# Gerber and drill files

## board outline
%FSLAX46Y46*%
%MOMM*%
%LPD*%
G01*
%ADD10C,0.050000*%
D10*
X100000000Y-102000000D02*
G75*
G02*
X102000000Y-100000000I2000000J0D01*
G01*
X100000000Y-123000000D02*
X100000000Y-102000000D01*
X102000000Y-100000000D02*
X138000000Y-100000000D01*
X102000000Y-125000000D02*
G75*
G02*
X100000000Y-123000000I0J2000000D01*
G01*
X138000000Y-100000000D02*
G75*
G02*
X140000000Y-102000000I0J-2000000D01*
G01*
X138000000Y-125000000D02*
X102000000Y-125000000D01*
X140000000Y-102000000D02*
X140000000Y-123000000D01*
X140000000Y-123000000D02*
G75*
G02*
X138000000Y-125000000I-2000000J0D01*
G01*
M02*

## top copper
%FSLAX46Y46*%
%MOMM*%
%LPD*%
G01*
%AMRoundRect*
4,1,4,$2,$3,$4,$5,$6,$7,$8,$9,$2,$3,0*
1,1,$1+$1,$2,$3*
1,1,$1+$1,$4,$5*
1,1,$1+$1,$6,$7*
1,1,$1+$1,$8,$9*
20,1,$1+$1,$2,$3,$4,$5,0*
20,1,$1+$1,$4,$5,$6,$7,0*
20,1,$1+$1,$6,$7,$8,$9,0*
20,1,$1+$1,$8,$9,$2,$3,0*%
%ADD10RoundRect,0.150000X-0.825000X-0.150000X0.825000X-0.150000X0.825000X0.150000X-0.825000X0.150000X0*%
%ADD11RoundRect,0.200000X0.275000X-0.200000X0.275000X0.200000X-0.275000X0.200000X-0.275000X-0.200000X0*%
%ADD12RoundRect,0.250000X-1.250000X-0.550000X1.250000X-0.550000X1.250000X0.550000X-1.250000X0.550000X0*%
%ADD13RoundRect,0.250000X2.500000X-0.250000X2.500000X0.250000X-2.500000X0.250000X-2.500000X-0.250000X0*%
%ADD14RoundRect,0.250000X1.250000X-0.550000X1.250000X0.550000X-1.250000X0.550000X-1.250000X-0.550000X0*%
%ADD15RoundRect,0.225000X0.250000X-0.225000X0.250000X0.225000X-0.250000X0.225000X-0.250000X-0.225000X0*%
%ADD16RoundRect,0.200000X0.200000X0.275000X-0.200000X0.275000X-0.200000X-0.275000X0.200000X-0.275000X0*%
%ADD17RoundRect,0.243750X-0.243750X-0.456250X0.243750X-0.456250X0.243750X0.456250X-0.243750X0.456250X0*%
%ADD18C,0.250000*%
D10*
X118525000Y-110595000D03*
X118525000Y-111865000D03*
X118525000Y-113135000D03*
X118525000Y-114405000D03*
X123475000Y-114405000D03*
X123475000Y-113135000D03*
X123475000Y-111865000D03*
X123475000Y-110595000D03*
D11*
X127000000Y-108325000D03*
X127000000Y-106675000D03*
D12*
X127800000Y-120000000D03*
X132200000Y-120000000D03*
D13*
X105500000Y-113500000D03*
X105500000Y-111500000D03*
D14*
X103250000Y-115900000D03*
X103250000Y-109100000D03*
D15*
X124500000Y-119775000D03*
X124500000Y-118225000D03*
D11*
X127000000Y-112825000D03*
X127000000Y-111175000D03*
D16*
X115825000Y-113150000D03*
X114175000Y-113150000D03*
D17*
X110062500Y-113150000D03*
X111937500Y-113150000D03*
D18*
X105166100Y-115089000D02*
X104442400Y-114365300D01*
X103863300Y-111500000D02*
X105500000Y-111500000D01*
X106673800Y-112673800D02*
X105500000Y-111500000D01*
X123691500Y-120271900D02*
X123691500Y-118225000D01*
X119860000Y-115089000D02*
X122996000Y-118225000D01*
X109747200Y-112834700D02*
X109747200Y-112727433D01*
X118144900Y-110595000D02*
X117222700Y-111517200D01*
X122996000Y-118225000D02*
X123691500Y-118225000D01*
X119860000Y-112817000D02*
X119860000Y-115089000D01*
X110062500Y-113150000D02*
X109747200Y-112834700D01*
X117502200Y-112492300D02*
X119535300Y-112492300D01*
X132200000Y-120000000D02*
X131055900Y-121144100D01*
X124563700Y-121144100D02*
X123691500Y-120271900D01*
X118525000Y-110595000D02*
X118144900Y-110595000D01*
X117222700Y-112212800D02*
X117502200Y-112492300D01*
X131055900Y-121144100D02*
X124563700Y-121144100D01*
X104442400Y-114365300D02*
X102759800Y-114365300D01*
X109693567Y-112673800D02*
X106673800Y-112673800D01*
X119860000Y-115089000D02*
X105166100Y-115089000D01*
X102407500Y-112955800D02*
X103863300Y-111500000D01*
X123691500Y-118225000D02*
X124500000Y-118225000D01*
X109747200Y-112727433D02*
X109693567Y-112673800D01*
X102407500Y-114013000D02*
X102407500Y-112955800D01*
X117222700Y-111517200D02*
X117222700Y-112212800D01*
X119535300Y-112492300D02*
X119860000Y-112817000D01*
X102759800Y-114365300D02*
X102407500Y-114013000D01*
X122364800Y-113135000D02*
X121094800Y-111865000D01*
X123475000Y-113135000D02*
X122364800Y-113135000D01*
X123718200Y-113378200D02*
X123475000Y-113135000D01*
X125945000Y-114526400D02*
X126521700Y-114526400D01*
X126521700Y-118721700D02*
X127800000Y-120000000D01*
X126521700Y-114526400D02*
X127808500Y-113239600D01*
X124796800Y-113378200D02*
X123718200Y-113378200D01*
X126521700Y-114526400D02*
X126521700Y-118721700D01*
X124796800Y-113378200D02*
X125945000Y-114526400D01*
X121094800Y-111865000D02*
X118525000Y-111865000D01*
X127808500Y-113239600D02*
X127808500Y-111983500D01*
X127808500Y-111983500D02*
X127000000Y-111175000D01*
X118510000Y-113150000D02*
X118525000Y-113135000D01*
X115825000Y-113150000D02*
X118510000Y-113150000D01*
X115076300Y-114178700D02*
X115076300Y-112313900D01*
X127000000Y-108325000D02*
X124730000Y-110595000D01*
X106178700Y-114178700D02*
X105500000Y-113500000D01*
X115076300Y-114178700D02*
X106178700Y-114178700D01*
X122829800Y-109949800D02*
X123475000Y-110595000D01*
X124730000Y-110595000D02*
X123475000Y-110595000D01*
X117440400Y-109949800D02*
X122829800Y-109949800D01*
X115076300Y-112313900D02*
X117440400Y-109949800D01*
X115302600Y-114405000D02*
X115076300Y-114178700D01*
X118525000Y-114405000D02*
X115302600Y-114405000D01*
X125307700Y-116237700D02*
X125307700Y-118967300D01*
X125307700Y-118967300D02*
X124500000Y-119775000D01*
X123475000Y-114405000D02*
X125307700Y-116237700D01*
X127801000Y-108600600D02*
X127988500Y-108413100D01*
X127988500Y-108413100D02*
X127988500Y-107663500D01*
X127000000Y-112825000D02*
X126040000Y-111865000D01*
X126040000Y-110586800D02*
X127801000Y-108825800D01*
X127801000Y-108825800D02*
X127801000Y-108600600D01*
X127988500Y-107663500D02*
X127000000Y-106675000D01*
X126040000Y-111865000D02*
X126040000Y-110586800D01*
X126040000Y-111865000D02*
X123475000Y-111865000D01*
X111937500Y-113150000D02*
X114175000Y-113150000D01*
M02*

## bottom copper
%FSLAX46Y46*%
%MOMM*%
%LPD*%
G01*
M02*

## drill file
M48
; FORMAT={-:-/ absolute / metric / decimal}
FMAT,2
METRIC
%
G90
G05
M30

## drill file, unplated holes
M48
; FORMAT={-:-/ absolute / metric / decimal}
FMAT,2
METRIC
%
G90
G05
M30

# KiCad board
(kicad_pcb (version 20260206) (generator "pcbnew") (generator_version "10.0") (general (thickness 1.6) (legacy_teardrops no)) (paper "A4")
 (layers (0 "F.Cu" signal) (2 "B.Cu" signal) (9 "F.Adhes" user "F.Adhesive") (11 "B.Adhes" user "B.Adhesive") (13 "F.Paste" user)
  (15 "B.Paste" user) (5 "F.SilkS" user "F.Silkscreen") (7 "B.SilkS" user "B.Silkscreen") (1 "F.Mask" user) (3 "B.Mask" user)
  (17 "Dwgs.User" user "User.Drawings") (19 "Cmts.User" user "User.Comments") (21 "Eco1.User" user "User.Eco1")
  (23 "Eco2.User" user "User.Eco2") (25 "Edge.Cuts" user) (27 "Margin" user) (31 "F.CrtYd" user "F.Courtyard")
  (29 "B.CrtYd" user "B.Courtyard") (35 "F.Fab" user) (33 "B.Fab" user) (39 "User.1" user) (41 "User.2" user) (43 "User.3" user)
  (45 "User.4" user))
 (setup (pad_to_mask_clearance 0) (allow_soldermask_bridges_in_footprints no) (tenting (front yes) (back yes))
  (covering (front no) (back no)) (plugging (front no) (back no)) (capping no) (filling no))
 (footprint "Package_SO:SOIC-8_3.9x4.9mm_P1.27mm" (layer "F.Cu") (at 121 112.5)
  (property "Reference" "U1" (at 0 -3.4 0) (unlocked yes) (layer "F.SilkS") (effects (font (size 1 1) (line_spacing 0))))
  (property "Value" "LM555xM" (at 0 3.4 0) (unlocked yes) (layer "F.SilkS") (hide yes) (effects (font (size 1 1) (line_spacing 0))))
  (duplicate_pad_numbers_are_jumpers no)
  (pad "1" smd roundrect (at -2.475 -1.905) (size 1.95 0.6) (layers "F.Cu" "F.Mask" "F.Paste") (roundrect_rratio 0.25) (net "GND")
   (zone_connect 0))
  (pad "2" smd roundrect (at -2.475 -0.635) (size 1.95 0.6) (layers "F.Cu" "F.Mask" "F.Paste") (roundrect_rratio 0.25)
   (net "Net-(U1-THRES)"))
  (pad "3" smd roundrect (at -2.475 0.635) (size 1.95 0.6) (layers "F.Cu" "F.Mask" "F.Paste") (roundrect_rratio 0.25) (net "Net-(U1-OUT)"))
  (pad "4" smd roundrect (at -2.475 1.905) (size 1.95 0.6) (layers "F.Cu" "F.Mask" "F.Paste") (roundrect_rratio 0.25) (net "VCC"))
  (pad "5" smd roundrect (at 2.475 1.905) (size 1.95 0.6) (layers "F.Cu" "F.Mask" "F.Paste") (roundrect_rratio 0.25) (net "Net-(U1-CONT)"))
  (pad "6" smd roundrect (at 2.475 0.635) (size 1.95 0.6) (layers "F.Cu" "F.Mask" "F.Paste") (roundrect_rratio 0.25) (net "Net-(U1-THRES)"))
  (pad "7" smd roundrect (at 2.475 -0.635) (size 1.95 0.6) (layers "F.Cu" "F.Mask" "F.Paste") (roundrect_rratio 0.25) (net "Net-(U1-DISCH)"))
  (pad "8" smd roundrect (at 2.475 -1.905) (size 1.95 0.6) (layers "F.Cu" "F.Mask" "F.Paste") (roundrect_rratio 0.25) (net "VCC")))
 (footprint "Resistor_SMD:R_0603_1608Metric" (layer "F.Cu") (at 127 107.5 90)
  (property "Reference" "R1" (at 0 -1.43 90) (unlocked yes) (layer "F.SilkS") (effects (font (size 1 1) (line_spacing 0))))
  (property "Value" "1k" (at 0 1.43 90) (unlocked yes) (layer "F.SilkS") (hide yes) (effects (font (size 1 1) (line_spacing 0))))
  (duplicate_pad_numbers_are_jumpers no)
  (pad "1" smd roundrect (at -0.825 0 90) (size 0.8 0.95) (layers "F.Cu" "F.Mask" "F.Paste") (roundrect_rratio 0.25) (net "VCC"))
  (pad "2" smd roundrect (at 0.825 0 90) (size 0.8 0.95) (layers "F.Cu" "F.Mask" "F.Paste") (roundrect_rratio 0.25) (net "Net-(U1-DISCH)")))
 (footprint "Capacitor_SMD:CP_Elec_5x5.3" (layer "F.Cu") (at 130 120)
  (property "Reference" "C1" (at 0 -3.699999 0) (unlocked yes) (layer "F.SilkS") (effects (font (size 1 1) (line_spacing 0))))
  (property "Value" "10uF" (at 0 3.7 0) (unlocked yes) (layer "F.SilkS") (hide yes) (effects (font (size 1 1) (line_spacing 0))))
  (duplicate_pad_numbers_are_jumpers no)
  (pad "1" smd roundrect (at -2.2 0) (size 3 1.6) (layers "F.Cu" "F.Mask" "F.Paste") (roundrect_rratio 0.15625) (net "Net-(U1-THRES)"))
  (pad "2" smd roundrect (at 2.2 0) (size 3 1.6) (layers "F.Cu" "F.Mask" "F.Paste") (roundrect_rratio 0.15625) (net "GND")))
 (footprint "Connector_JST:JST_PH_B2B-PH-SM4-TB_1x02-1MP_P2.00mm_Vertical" (layer "F.Cu") (at 105 112.5 90)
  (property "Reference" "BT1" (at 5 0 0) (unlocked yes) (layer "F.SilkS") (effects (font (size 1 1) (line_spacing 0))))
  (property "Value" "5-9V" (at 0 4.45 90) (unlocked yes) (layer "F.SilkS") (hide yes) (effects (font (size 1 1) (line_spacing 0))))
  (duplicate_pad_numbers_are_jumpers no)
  (pad "1" smd roundrect (at -1 0.5 90) (size 1 5.5) (layers "F.Cu" "F.Mask" "F.Paste") (roundrect_rratio 0.25) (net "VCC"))
  (pad "2" smd roundrect (at 1 0.5 90) (size 1 5.5) (layers "F.Cu" "F.Mask" "F.Paste") (roundrect_rratio 0.25) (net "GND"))
  (pad "MP" smd roundrect (at -3.4 -1.75 90) (size 1.6 3) (layers "F.Cu" "F.Mask" "F.Paste") (roundrect_rratio 0.15625))
  (pad "MP" smd roundrect (at 3.4 -1.75 90) (size 1.6 3) (layers "F.Cu" "F.Mask" "F.Paste") (roundrect_rratio 0.15625)))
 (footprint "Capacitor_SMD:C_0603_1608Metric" (layer "F.Cu") (at 124.5 119 90)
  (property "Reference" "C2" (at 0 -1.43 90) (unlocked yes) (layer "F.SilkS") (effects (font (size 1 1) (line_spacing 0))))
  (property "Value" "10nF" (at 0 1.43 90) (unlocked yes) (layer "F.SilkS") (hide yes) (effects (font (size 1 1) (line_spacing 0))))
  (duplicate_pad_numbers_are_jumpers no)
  (pad "1" smd roundrect (at -0.775 0 90) (size 0.9 0.95) (layers "F.Cu" "F.Mask" "F.Paste") (roundrect_rratio 0.25) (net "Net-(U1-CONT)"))
  (pad "2" smd roundrect (at 0.775 0 90) (size 0.9 0.95) (layers "F.Cu" "F.Mask" "F.Paste") (roundrect_rratio 0.25) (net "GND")))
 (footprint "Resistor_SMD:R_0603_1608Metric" (layer "F.Cu") (at 127 112 90)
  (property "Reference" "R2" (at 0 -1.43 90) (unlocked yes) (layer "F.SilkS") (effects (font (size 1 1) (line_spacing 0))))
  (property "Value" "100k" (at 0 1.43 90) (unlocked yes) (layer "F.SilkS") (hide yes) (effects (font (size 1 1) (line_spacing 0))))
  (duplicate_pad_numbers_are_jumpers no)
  (pad "1" smd roundrect (at -0.825 0 90) (size 0.8 0.95) (layers "F.Cu" "F.Mask" "F.Paste") (roundrect_rratio 0.25) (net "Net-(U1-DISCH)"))
  (pad "2" smd roundrect (at 0.825 0 90) (size 0.8 0.95) (layers "F.Cu" "F.Mask" "F.Paste") (roundrect_rratio 0.25) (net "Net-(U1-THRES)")))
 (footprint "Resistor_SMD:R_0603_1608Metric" (layer "F.Cu") (at 115 113.15 180)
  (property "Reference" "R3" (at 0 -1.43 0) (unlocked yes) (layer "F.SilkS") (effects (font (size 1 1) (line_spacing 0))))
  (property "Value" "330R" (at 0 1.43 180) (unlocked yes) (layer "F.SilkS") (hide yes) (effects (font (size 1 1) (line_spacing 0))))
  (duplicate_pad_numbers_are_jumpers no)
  (pad "1" smd roundrect (at -0.825 0 180) (size 0.8 0.95) (layers "F.Cu" "F.Mask" "F.Paste") (roundrect_rratio 0.25) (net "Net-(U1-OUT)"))
  (pad "2" smd roundrect (at 0.825 0 180) (size 0.8 0.95) (layers "F.Cu" "F.Mask" "F.Paste") (roundrect_rratio 0.25) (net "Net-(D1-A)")))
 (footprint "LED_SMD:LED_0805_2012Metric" (layer "F.Cu") (at 111 113.15)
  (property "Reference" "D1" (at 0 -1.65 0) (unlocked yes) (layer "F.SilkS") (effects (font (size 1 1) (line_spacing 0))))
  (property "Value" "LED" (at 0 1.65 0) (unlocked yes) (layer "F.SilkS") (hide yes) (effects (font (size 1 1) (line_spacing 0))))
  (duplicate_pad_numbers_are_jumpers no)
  (pad "1" smd roundrect (at -0.9375 0) (size 0.975 1.4) (layers "F.Cu" "F.Mask" "F.Paste") (roundrect_rratio 0.25) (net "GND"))
  (pad "2" smd roundrect (at 0.9375 0) (size 0.975 1.4) (layers "F.Cu" "F.Mask" "F.Paste") (roundrect_rratio 0.25) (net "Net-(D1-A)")))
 (gr_arc (start 100 102) (mid 100.585786 100.585786) (end 102 100) (stroke (width 0.05) (type default)) (layer "Edge.Cuts"))
 (gr_line (start 100 123) (end 100 102) (stroke (width 0.05) (type default)) (layer "Edge.Cuts"))
 (gr_line (start 102 100) (end 138 100) (stroke (width 0.05) (type default)) (layer "Edge.Cuts"))
 (gr_arc (start 102 125) (mid 100.585786 124.414213) (end 100 123) (stroke (width 0.05) (type default)) (layer "Edge.Cuts"))
 (gr_arc (start 138 100) (mid 139.414213 100.585786) (end 140 102) (stroke (width 0.05) (type default)) (layer "Edge.Cuts"))
 (gr_line (start 138 125) (end 102 125) (stroke (width 0.05) (type default)) (layer "Edge.Cuts"))
 (gr_line (start 140 102) (end 140 123) (stroke (width 0.05) (type default)) (layer "Edge.Cuts"))
 (gr_arc (start 140 123) (mid 139.414213 124.414213) (end 138 125) (stroke (width 0.05) (type default)) (layer "Edge.Cuts"))
 (segment (start 105.1661 115.089) (end 104.4424 114.3653) (width 0.25) (layer "F.Cu") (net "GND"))
 (segment (start 103.8633 111.5) (end 105.5 111.5) (width 0.25) (layer "F.Cu") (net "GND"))
 (segment (start 106.6738 112.6738) (end 105.5 111.5) (width 0.25) (layer "F.Cu") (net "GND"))
 (segment (start 123.6915 120.2719) (end 123.6915 118.225) (width 0.25) (layer "F.Cu") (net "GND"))
 (segment (start 119.86 115.089) (end 122.996 118.225) (width 0.25) (layer "F.Cu") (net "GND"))
 (segment (start 109.7472 112.8347) (end 109.747200 112.727433) (width 0.25) (layer "F.Cu") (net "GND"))
 (segment (start 118.1449 110.595) (end 117.2227 111.5172) (width 0.25) (layer "F.Cu") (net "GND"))
 (segment (start 122.996 118.225) (end 123.6915 118.225) (width 0.25) (layer "F.Cu") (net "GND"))
 (segment (start 119.86 112.817) (end 119.86 115.089) (width 0.25) (layer "F.Cu") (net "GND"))
 (segment (start 110.0625 113.15) (end 109.7472 112.8347) (width 0.25) (layer "F.Cu") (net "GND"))
 (segment (start 117.5022 112.4923) (end 119.5353 112.4923) (width 0.25) (layer "F.Cu") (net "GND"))
 (segment (start 132.2 120) (end 131.0559 121.1441) (width 0.25) (layer "F.Cu") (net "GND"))
 (segment (start 124.5637 121.1441) (end 123.6915 120.2719) (width 0.25) (layer "F.Cu") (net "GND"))
 (segment (start 118.525 110.595) (end 118.1449 110.595) (width 0.25) (layer "F.Cu") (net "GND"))
 (segment (start 117.2227 112.2128) (end 117.5022 112.4923) (width 0.25) (layer "F.Cu") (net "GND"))
 (segment (start 131.0559 121.1441) (end 124.5637 121.1441) (width 0.25) (layer "F.Cu") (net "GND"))
 (segment (start 104.4424 114.3653) (end 102.7598 114.3653) (width 0.25) (layer "F.Cu") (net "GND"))
 (segment (start 109.693567 112.673800) (end 106.6738 112.6738) (width 0.25) (layer "F.Cu") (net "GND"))
 (segment (start 119.86 115.089) (end 105.1661 115.089) (width 0.25) (layer "F.Cu") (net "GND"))
 (segment (start 102.4075 112.9558) (end 103.8633 111.5) (width 0.25) (layer "F.Cu") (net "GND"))
 (segment (start 123.6915 118.225) (end 124.5 118.225) (width 0.25) (layer "F.Cu") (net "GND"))
 (segment (start 102.4075 114.013) (end 102.4075 112.9558) (width 0.25) (layer "F.Cu") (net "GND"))
 (segment (start 117.2227 111.5172) (end 117.2227 112.2128) (width 0.25) (layer "F.Cu") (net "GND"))
 (segment (start 119.5353 112.4923) (end 119.86 112.817) (width 0.25) (layer "F.Cu") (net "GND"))
 (segment (start 102.7598 114.3653) (end 102.4075 114.013) (width 0.25) (layer "F.Cu") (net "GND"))
 (segment (start 122.3648 113.135) (end 121.0948 111.865) (width 0.25) (layer "F.Cu") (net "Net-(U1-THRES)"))
 (segment (start 123.475 113.135) (end 122.3648 113.135) (width 0.25) (layer "F.Cu") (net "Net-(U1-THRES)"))
 (segment (start 123.7182 113.3782) (end 123.475 113.135) (width 0.25) (layer "F.Cu") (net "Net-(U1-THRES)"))
 (segment (start 125.945 114.5264) (end 126.5217 114.5264) (width 0.25) (layer "F.Cu") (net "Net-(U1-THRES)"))
 (segment (start 126.5217 118.7217) (end 127.8 120) (width 0.25) (layer "F.Cu") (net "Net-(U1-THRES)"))
 (segment (start 126.5217 114.5264) (end 127.8085 113.2396) (width 0.25) (layer "F.Cu") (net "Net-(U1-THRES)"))
 (segment (start 124.7968 113.3782) (end 123.7182 113.3782) (width 0.25) (layer "F.Cu") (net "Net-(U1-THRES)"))
 (segment (start 126.5217 114.5264) (end 126.5217 118.7217) (width 0.25) (layer "F.Cu") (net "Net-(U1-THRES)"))
 (segment (start 124.7968 113.3782) (end 125.945 114.5264) (width 0.25) (layer "F.Cu") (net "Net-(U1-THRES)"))
 (segment (start 121.0948 111.865) (end 118.525 111.865) (width 0.25) (layer "F.Cu") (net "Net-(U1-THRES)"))
 (segment (start 127.8085 113.2396) (end 127.8085 111.9835) (width 0.25) (layer "F.Cu") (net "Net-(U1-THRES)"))
 (segment (start 127.8085 111.9835) (end 127 111.175) (width 0.25) (layer "F.Cu") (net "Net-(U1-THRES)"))
 (segment (start 118.51 113.15) (end 118.525 113.135) (width 0.25) (layer "F.Cu") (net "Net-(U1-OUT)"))
 (segment (start 115.825 113.15) (end 118.51 113.15) (width 0.25) (layer "F.Cu") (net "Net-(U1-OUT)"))
 (segment (start 115.0763 114.1787) (end 115.0763 112.3139) (width 0.25) (layer "F.Cu") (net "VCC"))
 (segment (start 127 108.325) (end 124.73 110.595) (width 0.25) (layer "F.Cu") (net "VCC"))
 (segment (start 106.1787 114.1787) (end 105.5 113.5) (width 0.25) (layer "F.Cu") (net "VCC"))
 (segment (start 115.0763 114.1787) (end 106.1787 114.1787) (width 0.25) (layer "F.Cu") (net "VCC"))
 (segment (start 122.8298 109.9498) (end 123.475 110.595) (width 0.25) (layer "F.Cu") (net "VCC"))
 (segment (start 124.73 110.595) (end 123.475 110.595) (width 0.25) (layer "F.Cu") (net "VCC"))
 (segment (start 117.4404 109.9498) (end 122.8298 109.9498) (width 0.25) (layer "F.Cu") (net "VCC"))
 (segment (start 115.0763 112.3139) (end 117.4404 109.9498) (width 0.25) (layer "F.Cu") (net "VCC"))
 (segment (start 115.3026 114.405) (end 115.0763 114.1787) (width 0.25) (layer "F.Cu") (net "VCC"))
 (segment (start 118.525 114.405) (end 115.3026 114.405) (width 0.25) (layer "F.Cu") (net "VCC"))
 (segment (start 125.3077 116.2377) (end 125.3077 118.9673) (width 0.25) (layer "F.Cu") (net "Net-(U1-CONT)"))
 (segment (start 125.3077 118.9673) (end 124.5 119.775) (width 0.25) (layer "F.Cu") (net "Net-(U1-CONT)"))
 (segment (start 123.475 114.405) (end 125.3077 116.2377) (width 0.25) (layer "F.Cu") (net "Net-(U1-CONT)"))
 (segment (start 127.801 108.6006) (end 127.9885 108.4131) (width 0.25) (layer "F.Cu") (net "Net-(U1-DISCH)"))
 (segment (start 127.9885 108.4131) (end 127.9885 107.6635) (width 0.25) (layer "F.Cu") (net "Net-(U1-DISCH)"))
 (segment (start 127 112.825) (end 126.04 111.865) (width 0.25) (layer "F.Cu") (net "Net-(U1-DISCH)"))
 (segment (start 126.04 110.5868) (end 127.801 108.8258) (width 0.25) (layer "F.Cu") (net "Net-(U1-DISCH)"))
 (segment (start 127.801 108.8258) (end 127.801 108.6006) (width 0.25) (layer "F.Cu") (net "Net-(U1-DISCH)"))
 (segment (start 127.9885 107.6635) (end 127 106.675) (width 0.25) (layer "F.Cu") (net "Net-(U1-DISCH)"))
 (segment (start 126.04 111.865) (end 126.04 110.5868) (width 0.25) (layer "F.Cu") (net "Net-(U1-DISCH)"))
 (segment (start 126.04 111.865) (end 123.475 111.865) (width 0.25) (layer "F.Cu") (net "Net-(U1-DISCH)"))
 (segment (start 111.9375 113.15) (end 114.175 113.15) (width 0.25) (layer "F.Cu") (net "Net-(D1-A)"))
 (segment (start 109.747200 112.727433) (end 109.693567 112.673800) (width 0.25) (layer "F.Cu") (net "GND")))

